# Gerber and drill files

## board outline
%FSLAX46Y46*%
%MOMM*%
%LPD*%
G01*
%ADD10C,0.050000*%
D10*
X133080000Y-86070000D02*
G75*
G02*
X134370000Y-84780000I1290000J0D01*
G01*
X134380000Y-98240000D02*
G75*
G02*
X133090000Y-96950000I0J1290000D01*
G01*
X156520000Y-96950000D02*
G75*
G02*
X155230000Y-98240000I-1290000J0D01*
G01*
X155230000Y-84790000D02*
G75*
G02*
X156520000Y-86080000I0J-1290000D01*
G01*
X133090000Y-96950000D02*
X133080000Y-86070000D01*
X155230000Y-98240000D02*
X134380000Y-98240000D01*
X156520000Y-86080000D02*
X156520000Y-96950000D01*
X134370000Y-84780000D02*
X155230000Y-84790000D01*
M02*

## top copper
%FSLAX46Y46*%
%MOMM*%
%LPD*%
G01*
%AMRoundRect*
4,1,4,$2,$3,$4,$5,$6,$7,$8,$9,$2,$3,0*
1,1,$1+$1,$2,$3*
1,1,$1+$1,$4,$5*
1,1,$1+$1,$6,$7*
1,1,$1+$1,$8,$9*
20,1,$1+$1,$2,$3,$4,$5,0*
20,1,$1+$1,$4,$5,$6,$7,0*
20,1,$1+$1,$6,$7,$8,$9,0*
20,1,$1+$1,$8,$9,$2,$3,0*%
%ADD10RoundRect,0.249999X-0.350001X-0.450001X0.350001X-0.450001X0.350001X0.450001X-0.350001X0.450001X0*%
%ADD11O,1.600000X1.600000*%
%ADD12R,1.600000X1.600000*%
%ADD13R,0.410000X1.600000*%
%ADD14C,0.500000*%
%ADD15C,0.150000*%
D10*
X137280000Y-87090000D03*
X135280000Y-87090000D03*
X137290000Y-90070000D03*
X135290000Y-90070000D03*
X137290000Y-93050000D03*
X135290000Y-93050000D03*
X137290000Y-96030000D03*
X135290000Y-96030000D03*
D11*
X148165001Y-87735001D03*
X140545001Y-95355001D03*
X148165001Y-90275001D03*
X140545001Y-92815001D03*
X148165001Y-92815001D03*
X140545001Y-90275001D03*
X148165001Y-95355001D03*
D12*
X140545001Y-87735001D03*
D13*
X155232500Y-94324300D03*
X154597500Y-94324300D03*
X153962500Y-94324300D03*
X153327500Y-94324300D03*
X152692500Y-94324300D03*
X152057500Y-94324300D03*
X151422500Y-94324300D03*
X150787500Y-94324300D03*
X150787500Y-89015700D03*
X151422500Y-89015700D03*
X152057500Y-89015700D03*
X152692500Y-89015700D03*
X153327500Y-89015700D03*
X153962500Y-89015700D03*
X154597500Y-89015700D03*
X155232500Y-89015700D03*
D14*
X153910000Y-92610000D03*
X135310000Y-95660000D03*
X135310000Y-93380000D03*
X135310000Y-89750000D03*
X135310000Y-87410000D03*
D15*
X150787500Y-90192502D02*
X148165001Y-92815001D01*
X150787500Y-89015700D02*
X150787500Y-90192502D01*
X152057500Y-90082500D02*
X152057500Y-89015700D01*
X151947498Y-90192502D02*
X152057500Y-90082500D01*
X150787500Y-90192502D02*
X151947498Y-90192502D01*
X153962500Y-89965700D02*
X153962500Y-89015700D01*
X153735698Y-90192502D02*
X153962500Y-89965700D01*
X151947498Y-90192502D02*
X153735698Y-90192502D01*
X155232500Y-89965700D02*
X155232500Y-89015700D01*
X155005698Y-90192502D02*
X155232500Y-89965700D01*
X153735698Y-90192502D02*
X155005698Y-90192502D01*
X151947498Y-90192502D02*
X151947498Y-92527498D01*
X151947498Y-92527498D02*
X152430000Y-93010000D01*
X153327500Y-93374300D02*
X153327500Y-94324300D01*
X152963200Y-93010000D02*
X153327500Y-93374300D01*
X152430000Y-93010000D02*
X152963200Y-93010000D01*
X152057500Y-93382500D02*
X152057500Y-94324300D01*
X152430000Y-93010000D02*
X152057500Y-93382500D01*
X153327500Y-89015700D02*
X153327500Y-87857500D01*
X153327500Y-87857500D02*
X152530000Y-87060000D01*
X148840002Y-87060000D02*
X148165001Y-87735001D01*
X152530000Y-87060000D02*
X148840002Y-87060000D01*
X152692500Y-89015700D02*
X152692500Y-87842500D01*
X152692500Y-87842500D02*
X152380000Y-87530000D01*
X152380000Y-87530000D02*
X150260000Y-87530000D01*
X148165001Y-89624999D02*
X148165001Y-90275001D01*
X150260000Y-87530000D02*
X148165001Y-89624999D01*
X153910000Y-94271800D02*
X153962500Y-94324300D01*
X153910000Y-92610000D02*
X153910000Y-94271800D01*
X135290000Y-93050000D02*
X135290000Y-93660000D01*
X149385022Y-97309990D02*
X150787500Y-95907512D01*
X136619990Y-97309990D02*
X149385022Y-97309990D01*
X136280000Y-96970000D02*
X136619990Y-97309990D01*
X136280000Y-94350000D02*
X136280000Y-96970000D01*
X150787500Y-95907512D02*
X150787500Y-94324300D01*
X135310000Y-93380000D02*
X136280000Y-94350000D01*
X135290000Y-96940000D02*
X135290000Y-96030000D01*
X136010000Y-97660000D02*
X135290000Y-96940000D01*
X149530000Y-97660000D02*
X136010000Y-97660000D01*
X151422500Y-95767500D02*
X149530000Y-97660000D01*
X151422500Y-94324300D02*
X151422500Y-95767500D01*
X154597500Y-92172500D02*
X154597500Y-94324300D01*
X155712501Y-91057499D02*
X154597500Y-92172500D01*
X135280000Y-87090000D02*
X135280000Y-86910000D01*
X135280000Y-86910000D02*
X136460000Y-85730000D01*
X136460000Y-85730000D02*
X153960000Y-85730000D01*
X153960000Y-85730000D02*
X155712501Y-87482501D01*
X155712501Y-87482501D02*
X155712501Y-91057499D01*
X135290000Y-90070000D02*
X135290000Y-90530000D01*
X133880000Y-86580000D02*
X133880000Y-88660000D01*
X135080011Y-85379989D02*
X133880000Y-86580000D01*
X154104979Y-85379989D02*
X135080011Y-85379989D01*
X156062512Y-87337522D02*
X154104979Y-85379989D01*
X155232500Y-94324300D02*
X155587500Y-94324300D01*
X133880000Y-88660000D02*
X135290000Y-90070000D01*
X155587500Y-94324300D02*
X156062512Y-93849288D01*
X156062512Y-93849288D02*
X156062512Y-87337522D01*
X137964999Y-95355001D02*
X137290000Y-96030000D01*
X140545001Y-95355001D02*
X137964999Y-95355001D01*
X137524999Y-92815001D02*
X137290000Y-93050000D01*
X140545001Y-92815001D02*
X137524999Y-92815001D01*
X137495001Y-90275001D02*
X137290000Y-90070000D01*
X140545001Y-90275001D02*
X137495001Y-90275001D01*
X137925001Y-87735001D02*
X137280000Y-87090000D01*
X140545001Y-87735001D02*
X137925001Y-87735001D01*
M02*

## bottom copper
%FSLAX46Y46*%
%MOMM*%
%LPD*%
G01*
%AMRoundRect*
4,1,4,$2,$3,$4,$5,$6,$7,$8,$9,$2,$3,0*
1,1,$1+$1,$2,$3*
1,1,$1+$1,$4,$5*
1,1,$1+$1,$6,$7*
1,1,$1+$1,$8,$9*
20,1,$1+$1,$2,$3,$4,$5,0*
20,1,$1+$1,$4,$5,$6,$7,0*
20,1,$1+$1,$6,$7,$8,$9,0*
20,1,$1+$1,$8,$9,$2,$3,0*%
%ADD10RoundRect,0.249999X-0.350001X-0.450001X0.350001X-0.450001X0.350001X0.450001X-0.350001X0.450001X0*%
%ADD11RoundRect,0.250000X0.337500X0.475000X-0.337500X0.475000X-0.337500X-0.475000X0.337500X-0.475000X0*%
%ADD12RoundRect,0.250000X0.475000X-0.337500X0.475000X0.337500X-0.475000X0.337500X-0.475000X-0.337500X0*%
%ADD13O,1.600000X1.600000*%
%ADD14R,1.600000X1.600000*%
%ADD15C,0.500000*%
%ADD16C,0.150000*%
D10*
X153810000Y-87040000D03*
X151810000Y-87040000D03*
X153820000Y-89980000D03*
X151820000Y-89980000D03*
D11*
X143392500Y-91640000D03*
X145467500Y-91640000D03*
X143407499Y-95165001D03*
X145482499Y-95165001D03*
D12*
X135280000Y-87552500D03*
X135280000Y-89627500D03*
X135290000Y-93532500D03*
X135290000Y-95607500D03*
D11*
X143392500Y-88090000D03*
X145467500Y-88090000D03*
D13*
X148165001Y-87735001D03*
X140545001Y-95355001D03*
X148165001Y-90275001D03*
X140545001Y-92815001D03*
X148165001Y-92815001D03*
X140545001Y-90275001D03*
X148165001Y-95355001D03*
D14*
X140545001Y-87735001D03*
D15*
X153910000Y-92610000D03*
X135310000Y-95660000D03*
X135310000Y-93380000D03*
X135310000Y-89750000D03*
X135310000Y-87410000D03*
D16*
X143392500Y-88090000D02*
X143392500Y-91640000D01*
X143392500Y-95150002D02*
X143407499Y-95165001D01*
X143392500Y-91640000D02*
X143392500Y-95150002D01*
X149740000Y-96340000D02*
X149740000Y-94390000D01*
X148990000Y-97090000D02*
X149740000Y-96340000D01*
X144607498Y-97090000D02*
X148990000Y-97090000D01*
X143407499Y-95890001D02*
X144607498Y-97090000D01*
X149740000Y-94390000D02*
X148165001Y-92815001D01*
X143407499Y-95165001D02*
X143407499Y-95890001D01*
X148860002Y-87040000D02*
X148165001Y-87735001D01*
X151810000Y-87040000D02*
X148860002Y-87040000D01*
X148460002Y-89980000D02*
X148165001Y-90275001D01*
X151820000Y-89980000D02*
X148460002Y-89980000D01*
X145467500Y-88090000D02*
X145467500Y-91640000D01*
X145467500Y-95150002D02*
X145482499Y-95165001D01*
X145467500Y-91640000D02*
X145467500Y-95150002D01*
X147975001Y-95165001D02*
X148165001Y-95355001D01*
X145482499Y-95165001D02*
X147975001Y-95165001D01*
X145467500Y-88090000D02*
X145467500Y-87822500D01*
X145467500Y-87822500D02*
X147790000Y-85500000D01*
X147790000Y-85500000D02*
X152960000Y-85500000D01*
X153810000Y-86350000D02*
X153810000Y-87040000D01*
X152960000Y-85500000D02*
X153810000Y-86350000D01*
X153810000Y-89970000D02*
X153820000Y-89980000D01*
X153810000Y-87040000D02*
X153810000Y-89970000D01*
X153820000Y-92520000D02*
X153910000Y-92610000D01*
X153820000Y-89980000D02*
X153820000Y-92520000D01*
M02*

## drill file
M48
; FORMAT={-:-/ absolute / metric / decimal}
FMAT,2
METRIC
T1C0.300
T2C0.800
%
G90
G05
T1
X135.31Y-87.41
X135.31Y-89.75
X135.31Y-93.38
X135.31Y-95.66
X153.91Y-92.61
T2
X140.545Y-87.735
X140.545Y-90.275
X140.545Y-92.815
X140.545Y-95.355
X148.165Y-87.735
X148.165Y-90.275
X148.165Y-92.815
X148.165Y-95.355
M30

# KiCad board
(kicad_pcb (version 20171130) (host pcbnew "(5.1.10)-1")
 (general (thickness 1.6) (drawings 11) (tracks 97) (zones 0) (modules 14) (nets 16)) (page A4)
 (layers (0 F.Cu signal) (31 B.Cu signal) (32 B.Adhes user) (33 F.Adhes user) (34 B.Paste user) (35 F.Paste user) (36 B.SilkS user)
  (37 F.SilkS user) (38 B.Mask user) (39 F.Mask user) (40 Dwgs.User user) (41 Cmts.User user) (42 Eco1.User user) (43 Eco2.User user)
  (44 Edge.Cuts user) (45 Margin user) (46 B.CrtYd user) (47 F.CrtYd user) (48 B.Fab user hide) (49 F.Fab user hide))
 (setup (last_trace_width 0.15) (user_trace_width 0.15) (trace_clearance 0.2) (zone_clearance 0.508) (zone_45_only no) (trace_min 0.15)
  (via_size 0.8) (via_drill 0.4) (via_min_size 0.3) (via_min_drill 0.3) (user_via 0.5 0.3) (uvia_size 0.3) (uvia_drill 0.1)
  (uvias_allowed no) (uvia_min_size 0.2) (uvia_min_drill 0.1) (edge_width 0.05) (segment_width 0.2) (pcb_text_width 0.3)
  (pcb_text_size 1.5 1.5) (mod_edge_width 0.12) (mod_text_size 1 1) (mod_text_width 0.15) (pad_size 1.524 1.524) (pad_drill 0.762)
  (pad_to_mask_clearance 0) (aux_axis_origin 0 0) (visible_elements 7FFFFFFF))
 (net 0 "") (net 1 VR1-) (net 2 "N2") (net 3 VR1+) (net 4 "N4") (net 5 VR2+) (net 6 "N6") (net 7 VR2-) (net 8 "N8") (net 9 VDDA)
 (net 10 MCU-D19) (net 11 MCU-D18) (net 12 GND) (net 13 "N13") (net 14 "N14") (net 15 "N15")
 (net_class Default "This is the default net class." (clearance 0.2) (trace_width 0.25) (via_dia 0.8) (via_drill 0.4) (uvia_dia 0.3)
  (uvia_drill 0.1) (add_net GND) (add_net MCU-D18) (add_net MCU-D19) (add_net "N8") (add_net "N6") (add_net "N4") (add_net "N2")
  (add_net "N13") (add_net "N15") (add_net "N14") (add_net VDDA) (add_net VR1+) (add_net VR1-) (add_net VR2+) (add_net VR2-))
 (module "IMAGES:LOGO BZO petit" (layer F.Cu) (at 144.7 91.8 305)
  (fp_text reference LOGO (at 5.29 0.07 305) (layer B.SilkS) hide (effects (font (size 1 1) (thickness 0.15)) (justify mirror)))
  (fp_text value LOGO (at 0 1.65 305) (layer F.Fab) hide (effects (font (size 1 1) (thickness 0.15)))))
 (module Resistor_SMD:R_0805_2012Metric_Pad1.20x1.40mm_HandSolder (layer F.Cu) (at 136.28 87.09)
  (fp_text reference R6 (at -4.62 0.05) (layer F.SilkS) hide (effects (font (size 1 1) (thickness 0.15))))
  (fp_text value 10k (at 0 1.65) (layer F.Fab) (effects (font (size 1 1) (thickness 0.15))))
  (pad 2 smd roundrect (at 1 0) (size 1.2 1.4) (layers F.Cu F.Paste F.Mask) (roundrect_rratio 0.2083325) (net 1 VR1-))
  (pad 1 smd roundrect (at -1 0) (size 1.2 1.4) (layers F.Cu F.Paste F.Mask) (roundrect_rratio 0.2083325) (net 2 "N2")))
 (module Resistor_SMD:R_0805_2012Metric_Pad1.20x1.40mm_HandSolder (layer F.Cu) (at 136.29 90.07)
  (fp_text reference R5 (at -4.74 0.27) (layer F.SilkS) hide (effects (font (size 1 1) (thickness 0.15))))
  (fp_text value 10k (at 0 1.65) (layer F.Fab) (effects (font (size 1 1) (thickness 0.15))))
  (pad 2 smd roundrect (at 1 0) (size 1.2 1.4) (layers F.Cu F.Paste F.Mask) (roundrect_rratio 0.2083325) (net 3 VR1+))
  (pad 1 smd roundrect (at -1 0) (size 1.2 1.4) (layers F.Cu F.Paste F.Mask) (roundrect_rratio 0.2083325) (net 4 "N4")))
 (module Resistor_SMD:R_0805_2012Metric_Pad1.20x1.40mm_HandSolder (layer F.Cu) (at 136.29 93.05)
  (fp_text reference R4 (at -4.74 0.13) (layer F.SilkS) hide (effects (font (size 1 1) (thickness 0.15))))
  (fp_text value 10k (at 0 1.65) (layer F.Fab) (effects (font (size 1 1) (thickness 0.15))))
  (pad 2 smd roundrect (at 1 0) (size 1.2 1.4) (layers F.Cu F.Paste F.Mask) (roundrect_rratio 0.2083325) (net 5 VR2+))
  (pad 1 smd roundrect (at -1 0) (size 1.2 1.4) (layers F.Cu F.Paste F.Mask) (roundrect_rratio 0.2083325) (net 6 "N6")))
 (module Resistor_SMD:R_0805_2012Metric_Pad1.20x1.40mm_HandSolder (layer F.Cu) (at 136.29 96.03)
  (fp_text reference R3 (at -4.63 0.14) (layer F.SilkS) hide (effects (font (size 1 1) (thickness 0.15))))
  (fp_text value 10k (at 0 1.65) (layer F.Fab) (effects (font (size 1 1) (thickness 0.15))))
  (pad 2 smd roundrect (at 1 0) (size 1.2 1.4) (layers F.Cu F.Paste F.Mask) (roundrect_rratio 0.2083325) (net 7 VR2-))
  (pad 1 smd roundrect (at -1 0) (size 1.2 1.4) (layers F.Cu F.Paste F.Mask) (roundrect_rratio 0.2083325) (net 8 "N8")))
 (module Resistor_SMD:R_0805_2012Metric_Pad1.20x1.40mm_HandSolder (layer B.Cu) (at 152.81 87.04)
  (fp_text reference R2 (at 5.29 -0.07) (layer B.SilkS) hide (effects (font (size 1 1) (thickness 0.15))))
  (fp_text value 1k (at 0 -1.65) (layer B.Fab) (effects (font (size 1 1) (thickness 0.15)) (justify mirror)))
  (pad 2 smd roundrect (at 1 0) (size 1.2 1.4) (layers B.Cu B.Paste B.Mask) (roundrect_rratio 0.2083325) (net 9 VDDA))
  (pad 1 smd roundrect (at -1 0) (size 1.2 1.4) (layers B.Cu B.Paste B.Mask) (roundrect_rratio 0.2083325) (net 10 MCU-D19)))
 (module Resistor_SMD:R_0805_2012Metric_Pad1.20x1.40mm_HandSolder (layer B.Cu) (at 152.82 89.98)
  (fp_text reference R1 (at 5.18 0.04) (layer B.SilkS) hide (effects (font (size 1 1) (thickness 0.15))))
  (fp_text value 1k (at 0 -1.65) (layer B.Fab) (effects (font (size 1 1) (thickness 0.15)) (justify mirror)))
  (pad 2 smd roundrect (at 1 0) (size 1.2 1.4) (layers B.Cu B.Paste B.Mask) (roundrect_rratio 0.2083325) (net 9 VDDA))
  (pad 1 smd roundrect (at -1 0) (size 1.2 1.4) (layers B.Cu B.Paste B.Mask) (roundrect_rratio 0.2083325) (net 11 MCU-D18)))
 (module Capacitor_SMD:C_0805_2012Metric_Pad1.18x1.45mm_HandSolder (layer B.Cu) (at 144.43 91.64 180)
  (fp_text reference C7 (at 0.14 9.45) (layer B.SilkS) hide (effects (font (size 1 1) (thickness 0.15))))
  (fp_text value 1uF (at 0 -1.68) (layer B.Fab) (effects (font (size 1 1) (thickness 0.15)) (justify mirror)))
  (pad 2 smd roundrect (at 1.0375 0 180) (size 1.175 1.45) (layers B.Cu B.Paste B.Mask) (roundrect_rratio 0.2127659574468085) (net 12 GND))
  (pad 1 smd roundrect (at -1.0375 0 180) (size 1.175 1.45) (layers B.Cu B.Paste B.Mask) (roundrect_rratio 0.2127659574468085) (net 9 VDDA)))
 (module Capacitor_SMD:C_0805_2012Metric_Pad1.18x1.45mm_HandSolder (layer B.Cu) (at 144.444999 95.165001 180)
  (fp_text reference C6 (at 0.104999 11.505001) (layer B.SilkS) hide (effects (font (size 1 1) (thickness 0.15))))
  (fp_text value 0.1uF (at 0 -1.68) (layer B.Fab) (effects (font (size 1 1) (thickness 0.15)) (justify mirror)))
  (pad 2 smd roundrect (at 1.0375 0 180) (size 1.175 1.45) (layers B.Cu B.Paste B.Mask) (roundrect_rratio 0.2127659574468085) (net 12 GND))
  (pad 1 smd roundrect (at -1.0375 0 180) (size 1.175 1.45) (layers B.Cu B.Paste B.Mask) (roundrect_rratio 0.2127659574468085) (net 9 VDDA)))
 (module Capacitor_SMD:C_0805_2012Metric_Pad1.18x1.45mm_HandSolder (layer B.Cu) (at 135.28 88.59 90)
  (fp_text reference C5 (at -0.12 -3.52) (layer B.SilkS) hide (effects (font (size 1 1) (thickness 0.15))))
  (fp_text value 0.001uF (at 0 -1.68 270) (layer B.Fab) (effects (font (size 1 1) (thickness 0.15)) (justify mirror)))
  (pad 2 smd roundrect (at 1.0375 0 90) (size 1.175 1.45) (layers B.Cu B.Paste B.Mask) (roundrect_rratio 0.2127659574468085) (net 2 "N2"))
  (pad 1 smd roundrect (at -1.0375 0 90) (size 1.175 1.45) (layers B.Cu B.Paste B.Mask) (roundrect_rratio 0.2127659574468085) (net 4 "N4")))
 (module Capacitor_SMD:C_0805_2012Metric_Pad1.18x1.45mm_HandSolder (layer B.Cu) (at 135.29 94.57 90)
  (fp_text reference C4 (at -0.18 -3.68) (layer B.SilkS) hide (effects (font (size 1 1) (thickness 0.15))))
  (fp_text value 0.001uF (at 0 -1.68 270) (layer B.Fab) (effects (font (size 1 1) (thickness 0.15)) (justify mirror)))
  (pad 2 smd roundrect (at 1.0375 0 90) (size 1.175 1.45) (layers B.Cu B.Paste B.Mask) (roundrect_rratio 0.2127659574468085) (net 6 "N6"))
  (pad 1 smd roundrect (at -1.0375 0 90) (size 1.175 1.45) (layers B.Cu B.Paste B.Mask) (roundrect_rratio 0.2127659574468085) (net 8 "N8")))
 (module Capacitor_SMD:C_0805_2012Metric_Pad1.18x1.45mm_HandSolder (layer B.Cu) (at 144.43 88.09 180)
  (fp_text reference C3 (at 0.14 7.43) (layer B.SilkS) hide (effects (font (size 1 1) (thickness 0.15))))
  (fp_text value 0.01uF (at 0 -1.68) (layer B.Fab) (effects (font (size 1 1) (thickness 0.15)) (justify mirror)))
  (pad 2 smd roundrect (at 1.0375 0 180) (size 1.175 1.45) (layers B.Cu B.Paste B.Mask) (roundrect_rratio 0.2127659574468085) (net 12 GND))
  (pad 1 smd roundrect (at -1.0375 0 180) (size 1.175 1.45) (layers B.Cu B.Paste B.Mask) (roundrect_rratio 0.2127659574468085) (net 9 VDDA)))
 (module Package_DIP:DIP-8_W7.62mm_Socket (layer F.Cu) (at 140.545001 87.735001)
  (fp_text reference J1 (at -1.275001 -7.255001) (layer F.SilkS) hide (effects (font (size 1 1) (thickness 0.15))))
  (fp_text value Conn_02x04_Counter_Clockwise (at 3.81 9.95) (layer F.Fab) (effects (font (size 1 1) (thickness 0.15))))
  (pad 8 thru_hole oval (at 7.62 0) (size 1.6 1.6) (drill 0.8) (layers *.Cu *.Mask) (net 10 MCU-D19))
  (pad 4 thru_hole oval (at 0 7.62) (size 1.6 1.6) (drill 0.8) (layers *.Cu *.Mask) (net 7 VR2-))
  (pad 7 thru_hole oval (at 7.62 2.54) (size 1.6 1.6) (drill 0.8) (layers *.Cu *.Mask) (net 11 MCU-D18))
  (pad 3 thru_hole oval (at 0 5.08) (size 1.6 1.6) (drill 0.8) (layers *.Cu *.Mask) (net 5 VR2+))
  (pad 6 thru_hole oval (at 7.62 5.08) (size 1.6 1.6) (drill 0.8) (layers *.Cu *.Mask) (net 12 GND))
  (pad 2 thru_hole oval (at 0 2.54) (size 1.6 1.6) (drill 0.8) (layers *.Cu *.Mask) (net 3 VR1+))
  (pad 5 thru_hole oval (at 7.62 7.62) (size 1.6 1.6) (drill 0.8) (layers *.Cu *.Mask) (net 9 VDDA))
  (pad 1 thru_hole rect (at 0 0) (size 1.6 1.6) (drill 0.8) (layers *.Cu *.Mask) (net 1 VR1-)))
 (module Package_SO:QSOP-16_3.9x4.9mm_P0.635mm (layer F.Cu) (at 153.01 91.67 270)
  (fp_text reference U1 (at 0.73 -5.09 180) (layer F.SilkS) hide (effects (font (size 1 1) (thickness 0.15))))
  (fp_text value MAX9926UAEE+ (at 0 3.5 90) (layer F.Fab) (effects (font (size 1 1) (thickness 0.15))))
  (pad 16 smd rect (at 2.6543 -2.2225 270) (size 1.6 0.41) (layers F.Cu F.Paste F.Mask) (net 4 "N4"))
  (pad 15 smd rect (at 2.6543 -1.5875 270) (size 1.6 0.41) (layers F.Cu F.Paste F.Mask) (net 2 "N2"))
  (pad 14 smd rect (at 2.6543 -0.9525 270) (size 1.6 0.41) (layers F.Cu F.Paste F.Mask) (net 9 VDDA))
  (pad 13 smd rect (at 2.6543 -0.3175 270) (size 1.6 0.41) (layers F.Cu F.Paste F.Mask) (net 12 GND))
  (pad 12 smd rect (at 2.6543 0.3175 270) (size 1.6 0.41) (layers F.Cu F.Paste F.Mask) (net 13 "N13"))
  (pad 11 smd rect (at 2.6543 0.9525 270) (size 1.6 0.41) (layers F.Cu F.Paste F.Mask) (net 12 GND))
  (pad 10 smd rect (at 2.6543 1.5875 270) (size 1.6 0.41) (layers F.Cu F.Paste F.Mask) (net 8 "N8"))
  (pad 9 smd rect (at 2.6543 2.2225 270) (size 1.6 0.41) (layers F.Cu F.Paste F.Mask) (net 6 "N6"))
  (pad 8 smd rect (at -2.6543 2.2225 270) (size 1.6 0.41) (layers F.Cu F.Paste F.Mask) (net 12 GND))
  (pad 7 smd rect (at -2.6543 1.5875 270) (size 1.6 0.41) (layers F.Cu F.Paste F.Mask) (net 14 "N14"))
  (pad 6 smd rect (at -2.6543 0.9525 270) (size 1.6 0.41) (layers F.Cu F.Paste F.Mask) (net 12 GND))
  (pad 5 smd rect (at -2.6543 0.3175 270) (size 1.6 0.41) (layers F.Cu F.Paste F.Mask) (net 11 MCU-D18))
  (pad 4 smd rect (at -2.6543 -0.3175 270) (size 1.6 0.41) (layers F.Cu F.Paste F.Mask) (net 10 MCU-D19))
  (pad 3 smd rect (at -2.6543 -0.9525 270) (size 1.6 0.41) (layers F.Cu F.Paste F.Mask) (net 12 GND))
  (pad 2 smd rect (at -2.6543 -1.5875 270) (size 1.6 0.41) (layers F.Cu F.Paste F.Mask) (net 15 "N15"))
  (pad 1 smd rect (at -2.6543 -2.2225 270) (size 1.6 0.41) (layers F.Cu F.Paste F.Mask) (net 12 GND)))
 (gr_arc (start 134.37 86.07) (end 134.37 84.78) (angle -90) (layer Edge.Cuts) (width 0.05))
 (gr_arc (start 134.38 96.95) (end 133.09 96.95) (angle -90) (layer Edge.Cuts) (width 0.05))
 (gr_arc (start 155.23 96.95) (end 155.23 98.24) (angle -90) (layer Edge.Cuts) (width 0.05))
 (gr_arc (start 155.23 86.08) (end 156.52 86.08) (angle -90) (layer Edge.Cuts) (width 0.05))
 (gr_line (start 133.09 96.95) (end 133.08 86.07) (layer Edge.Cuts) (width 0.05))
 (gr_line (start 155.23 98.24) (end 134.38 98.24) (layer Edge.Cuts) (width 0.05))
 (gr_line (start 156.52 86.08) (end 156.52 96.95) (layer Edge.Cuts) (width 0.05))
 (gr_line (start 134.37 84.78) (end 155.23 84.79) (layer Edge.Cuts) (width 0.05))
 (segment (start 143.3925 88.09) (end 143.3925 91.64) (width 0.15) (layer B.Cu) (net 12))
 (segment (start 143.3925 95.150002) (end 143.407499 95.165001) (width 0.15) (layer B.Cu) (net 12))
 (segment (start 143.3925 91.64) (end 143.3925 95.150002) (width 0.15) (layer B.Cu) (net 12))
 (segment (start 150.7875 90.192502) (end 148.165001 92.815001) (width 0.15) (layer F.Cu) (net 12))
 (segment (start 150.7875 89.0157) (end 150.7875 90.192502) (width 0.15) (layer F.Cu) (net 12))
 (segment (start 152.0575 90.0825) (end 152.0575 89.0157) (width 0.15) (layer F.Cu) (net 12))
 (segment (start 151.947498 90.192502) (end 152.0575 90.0825) (width 0.15) (layer F.Cu) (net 12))
 (segment (start 150.7875 90.192502) (end 151.947498 90.192502) (width 0.15) (layer F.Cu) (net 12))
 (segment (start 153.9625 89.9657) (end 153.9625 89.0157) (width 0.15) (layer F.Cu) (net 12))
 (segment (start 153.735698 90.192502) (end 153.9625 89.9657) (width 0.15) (layer F.Cu) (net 12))
 (segment (start 151.947498 90.192502) (end 153.735698 90.192502) (width 0.15) (layer F.Cu) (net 12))
 (segment (start 155.2325 89.9657) (end 155.2325 89.0157) (width 0.15) (layer F.Cu) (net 12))
 (segment (start 155.005698 90.192502) (end 155.2325 89.9657) (width 0.15) (layer F.Cu) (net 12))
 (segment (start 153.735698 90.192502) (end 155.005698 90.192502) (width 0.15) (layer F.Cu) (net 12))
 (segment (start 151.947498 90.192502) (end 151.947498 92.527498) (width 0.15) (layer F.Cu) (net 12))
 (segment (start 151.947498 92.527498) (end 152.43 93.01) (width 0.15) (layer F.Cu) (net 12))
 (segment (start 153.3275 93.3743) (end 153.3275 94.3243) (width 0.15) (layer F.Cu) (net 12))
 (segment (start 152.9632 93.01) (end 153.3275 93.3743) (width 0.15) (layer F.Cu) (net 12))
 (segment (start 152.43 93.01) (end 152.9632 93.01) (width 0.15) (layer F.Cu) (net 12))
 (segment (start 152.0575 93.3825) (end 152.0575 94.3243) (width 0.15) (layer F.Cu) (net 12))
 (segment (start 152.43 93.01) (end 152.0575 93.3825) (width 0.15) (layer F.Cu) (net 12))
 (segment (start 149.74 96.34) (end 149.74 94.39) (width 0.15) (layer B.Cu) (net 12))
 (segment (start 148.99 97.09) (end 149.74 96.34) (width 0.15) (layer B.Cu) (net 12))
 (segment (start 144.607498 97.09) (end 148.99 97.09) (width 0.15) (layer B.Cu) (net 12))
 (segment (start 143.407499 95.890001) (end 144.607498 97.09) (width 0.15) (layer B.Cu) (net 12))
 (segment (start 149.74 94.39) (end 148.165001 92.815001) (width 0.15) (layer B.Cu) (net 12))
 (segment (start 143.407499 95.165001) (end 143.407499 95.890001) (width 0.15) (layer B.Cu) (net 12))
 (segment (start 148.860002 87.04) (end 148.165001 87.735001) (width 0.15) (layer B.Cu) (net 10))
 (segment (start 151.81 87.04) (end 148.860002 87.04) (width 0.15) (layer B.Cu) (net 10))
 (segment (start 153.3275 89.0157) (end 153.3275 87.8575) (width 0.15) (layer F.Cu) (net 10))
 (segment (start 153.3275 87.8575) (end 152.53 87.06) (width 0.15) (layer F.Cu) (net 10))
 (segment (start 148.840002 87.06) (end 148.165001 87.735001) (width 0.15) (layer F.Cu) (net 10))
 (segment (start 152.53 87.06) (end 148.840002 87.06) (width 0.15) (layer F.Cu) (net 10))
 (segment (start 148.460002 89.98) (end 148.165001 90.275001) (width 0.15) (layer B.Cu) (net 11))
 (segment (start 151.82 89.98) (end 148.460002 89.98) (width 0.15) (layer B.Cu) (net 11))
 (segment (start 152.6925 89.0157) (end 152.6925 87.8425) (width 0.15) (layer F.Cu) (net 11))
 (segment (start 152.6925 87.8425) (end 152.38 87.53) (width 0.15) (layer F.Cu) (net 11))
 (segment (start 152.38 87.53) (end 150.26 87.53) (width 0.15) (layer F.Cu) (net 11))
 (segment (start 148.165001 89.624999) (end 148.165001 90.275001) (width 0.15) (layer F.Cu) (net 11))
 (segment (start 150.26 87.53) (end 148.165001 89.624999) (width 0.15) (layer F.Cu) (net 11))
 (segment (start 145.4675 88.09) (end 145.4675 91.64) (width 0.15) (layer B.Cu) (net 9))
 (segment (start 145.4675 95.150002) (end 145.482499 95.165001) (width 0.15) (layer B.Cu) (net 9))
 (segment (start 145.4675 91.64) (end 145.4675 95.150002) (width 0.15) (layer B.Cu) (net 9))
 (segment (start 147.975001 95.165001) (end 148.165001 95.355001) (width 0.15) (layer B.Cu) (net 9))
 (segment (start 145.482499 95.165001) (end 147.975001 95.165001) (width 0.15) (layer B.Cu) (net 9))
 (segment (start 145.4675 88.09) (end 145.4675 87.8225) (width 0.15) (layer B.Cu) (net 9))
 (segment (start 145.4675 87.8225) (end 147.79 85.5) (width 0.15) (layer B.Cu) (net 9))
 (segment (start 147.79 85.5) (end 152.96 85.5) (width 0.15) (layer B.Cu) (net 9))
 (segment (start 153.81 86.35) (end 153.81 87.04) (width 0.15) (layer B.Cu) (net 9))
 (segment (start 152.96 85.5) (end 153.81 86.35) (width 0.15) (layer B.Cu) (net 9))
 (segment (start 153.81 89.97) (end 153.82 89.98) (width 0.15) (layer B.Cu) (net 9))
 (segment (start 153.81 87.04) (end 153.81 89.97) (width 0.15) (layer B.Cu) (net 9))
 (via (at 153.91 92.61) (size 0.5) (drill 0.3) (layers F.Cu B.Cu) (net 9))
 (segment (start 153.82 92.52) (end 153.91 92.61) (width 0.15) (layer B.Cu) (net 9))
 (segment (start 153.82 89.98) (end 153.82 92.52) (width 0.15) (layer B.Cu) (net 9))
 (segment (start 153.91 94.2718) (end 153.9625 94.3243) (width 0.15) (layer F.Cu) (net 9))
 (segment (start 153.91 92.61) (end 153.91 94.2718) (width 0.15) (layer F.Cu) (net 9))
 (via (at 135.31 95.66) (size 0.5) (drill 0.3) (layers F.Cu B.Cu) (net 8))
 (via (at 135.31 93.38) (size 0.5) (drill 0.3) (layers F.Cu B.Cu) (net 6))
 (segment (start 135.29 93.05) (end 135.29 93.66) (width 0.15) (layer F.Cu) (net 6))
 (segment (start 149.385022 97.30999) (end 150.7875 95.907512) (width 0.15) (layer F.Cu) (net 6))
 (segment (start 136.61999 97.30999) (end 149.385022 97.30999) (width 0.15) (layer F.Cu) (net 6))
 (segment (start 136.28 96.97) (end 136.61999 97.30999) (width 0.15) (layer F.Cu) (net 6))
 (segment (start 136.28 94.35) (end 136.28 96.97) (width 0.15) (layer F.Cu) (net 6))
 (segment (start 150.7875 95.907512) (end 150.7875 94.3243) (width 0.15) (layer F.Cu) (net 6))
 (segment (start 135.31 93.38) (end 136.28 94.35) (width 0.15) (layer F.Cu) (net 6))
 (segment (start 135.29 96.94) (end 135.29 96.03) (width 0.15) (layer F.Cu) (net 8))
 (segment (start 136.01 97.66) (end 135.29 96.94) (width 0.15) (layer F.Cu) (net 8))
 (segment (start 149.53 97.66) (end 136.01 97.66) (width 0.15) (layer F.Cu) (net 8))
 (segment (start 151.4225 95.7675) (end 149.53 97.66) (width 0.15) (layer F.Cu) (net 8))
 (segment (start 151.4225 94.3243) (end 151.4225 95.7675) (width 0.15) (layer F.Cu) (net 8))
 (via (at 135.31 89.75) (size 0.5) (drill 0.3) (layers F.Cu B.Cu) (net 4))
 (via (at 135.31 87.41) (size 0.5) (drill 0.3) (layers F.Cu B.Cu) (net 2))
 (segment (start 154.5975 92.1725) (end 154.5975 94.3243) (width 0.15) (layer F.Cu) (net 2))
 (segment (start 155.712501 91.057499) (end 154.5975 92.1725) (width 0.15) (layer F.Cu) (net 2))
 (segment (start 135.28 87.09) (end 135.28 86.91) (width 0.15) (layer F.Cu) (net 2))
 (segment (start 135.28 86.91) (end 136.46 85.73) (width 0.15) (layer F.Cu) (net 2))
 (segment (start 136.46 85.73) (end 153.96 85.73) (width 0.15) (layer F.Cu) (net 2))
 (segment (start 153.96 85.73) (end 155.712501 87.482501) (width 0.15) (layer F.Cu) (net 2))
 (segment (start 155.712501 87.482501) (end 155.712501 91.057499) (width 0.15) (layer F.Cu) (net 2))
 (segment (start 135.29 90.07) (end 135.29 90.53) (width 0.15) (layer F.Cu) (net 4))
 (segment (start 133.88 86.58) (end 133.88 88.66) (width 0.15) (layer F.Cu) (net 4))
 (segment (start 135.080011 85.379989) (end 133.88 86.58) (width 0.15) (layer F.Cu) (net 4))
 (segment (start 154.104979 85.379989) (end 135.080011 85.379989) (width 0.15) (layer F.Cu) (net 4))
 (segment (start 156.062512 87.337522) (end 154.104979 85.379989) (width 0.15) (layer F.Cu) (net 4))
 (segment (start 155.2325 94.3243) (end 155.5875 94.3243) (width 0.15) (layer F.Cu) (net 4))
 (segment (start 133.88 88.66) (end 135.29 90.07) (width 0.15) (layer F.Cu) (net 4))
 (segment (start 155.5875 94.3243) (end 156.062512 93.849288) (width 0.15) (layer F.Cu) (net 4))
 (segment (start 156.062512 93.849288) (end 156.062512 87.337522) (width 0.15) (layer F.Cu) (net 4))
 (segment (start 137.964999 95.355001) (end 137.29 96.03) (width 0.15) (layer F.Cu) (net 7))
 (segment (start 140.545001 95.355001) (end 137.964999 95.355001) (width 0.15) (layer F.Cu) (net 7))
 (segment (start 137.524999 92.815001) (end 137.29 93.05) (width 0.15) (layer F.Cu) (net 5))
 (segment (start 140.545001 92.815001) (end 137.524999 92.815001) (width 0.15) (layer F.Cu) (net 5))
 (segment (start 137.495001 90.275001) (end 137.29 90.07) (width 0.15) (layer F.Cu) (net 3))
 (segment (start 140.545001 90.275001) (end 137.495001 90.275001) (width 0.15) (layer F.Cu) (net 3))
 (segment (start 137.925001 87.735001) (end 137.28 87.09) (width 0.15) (layer F.Cu) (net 1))
 (segment (start 140.545001 87.735001) (end 137.925001 87.735001) (width 0.15) (layer F.Cu) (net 1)))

